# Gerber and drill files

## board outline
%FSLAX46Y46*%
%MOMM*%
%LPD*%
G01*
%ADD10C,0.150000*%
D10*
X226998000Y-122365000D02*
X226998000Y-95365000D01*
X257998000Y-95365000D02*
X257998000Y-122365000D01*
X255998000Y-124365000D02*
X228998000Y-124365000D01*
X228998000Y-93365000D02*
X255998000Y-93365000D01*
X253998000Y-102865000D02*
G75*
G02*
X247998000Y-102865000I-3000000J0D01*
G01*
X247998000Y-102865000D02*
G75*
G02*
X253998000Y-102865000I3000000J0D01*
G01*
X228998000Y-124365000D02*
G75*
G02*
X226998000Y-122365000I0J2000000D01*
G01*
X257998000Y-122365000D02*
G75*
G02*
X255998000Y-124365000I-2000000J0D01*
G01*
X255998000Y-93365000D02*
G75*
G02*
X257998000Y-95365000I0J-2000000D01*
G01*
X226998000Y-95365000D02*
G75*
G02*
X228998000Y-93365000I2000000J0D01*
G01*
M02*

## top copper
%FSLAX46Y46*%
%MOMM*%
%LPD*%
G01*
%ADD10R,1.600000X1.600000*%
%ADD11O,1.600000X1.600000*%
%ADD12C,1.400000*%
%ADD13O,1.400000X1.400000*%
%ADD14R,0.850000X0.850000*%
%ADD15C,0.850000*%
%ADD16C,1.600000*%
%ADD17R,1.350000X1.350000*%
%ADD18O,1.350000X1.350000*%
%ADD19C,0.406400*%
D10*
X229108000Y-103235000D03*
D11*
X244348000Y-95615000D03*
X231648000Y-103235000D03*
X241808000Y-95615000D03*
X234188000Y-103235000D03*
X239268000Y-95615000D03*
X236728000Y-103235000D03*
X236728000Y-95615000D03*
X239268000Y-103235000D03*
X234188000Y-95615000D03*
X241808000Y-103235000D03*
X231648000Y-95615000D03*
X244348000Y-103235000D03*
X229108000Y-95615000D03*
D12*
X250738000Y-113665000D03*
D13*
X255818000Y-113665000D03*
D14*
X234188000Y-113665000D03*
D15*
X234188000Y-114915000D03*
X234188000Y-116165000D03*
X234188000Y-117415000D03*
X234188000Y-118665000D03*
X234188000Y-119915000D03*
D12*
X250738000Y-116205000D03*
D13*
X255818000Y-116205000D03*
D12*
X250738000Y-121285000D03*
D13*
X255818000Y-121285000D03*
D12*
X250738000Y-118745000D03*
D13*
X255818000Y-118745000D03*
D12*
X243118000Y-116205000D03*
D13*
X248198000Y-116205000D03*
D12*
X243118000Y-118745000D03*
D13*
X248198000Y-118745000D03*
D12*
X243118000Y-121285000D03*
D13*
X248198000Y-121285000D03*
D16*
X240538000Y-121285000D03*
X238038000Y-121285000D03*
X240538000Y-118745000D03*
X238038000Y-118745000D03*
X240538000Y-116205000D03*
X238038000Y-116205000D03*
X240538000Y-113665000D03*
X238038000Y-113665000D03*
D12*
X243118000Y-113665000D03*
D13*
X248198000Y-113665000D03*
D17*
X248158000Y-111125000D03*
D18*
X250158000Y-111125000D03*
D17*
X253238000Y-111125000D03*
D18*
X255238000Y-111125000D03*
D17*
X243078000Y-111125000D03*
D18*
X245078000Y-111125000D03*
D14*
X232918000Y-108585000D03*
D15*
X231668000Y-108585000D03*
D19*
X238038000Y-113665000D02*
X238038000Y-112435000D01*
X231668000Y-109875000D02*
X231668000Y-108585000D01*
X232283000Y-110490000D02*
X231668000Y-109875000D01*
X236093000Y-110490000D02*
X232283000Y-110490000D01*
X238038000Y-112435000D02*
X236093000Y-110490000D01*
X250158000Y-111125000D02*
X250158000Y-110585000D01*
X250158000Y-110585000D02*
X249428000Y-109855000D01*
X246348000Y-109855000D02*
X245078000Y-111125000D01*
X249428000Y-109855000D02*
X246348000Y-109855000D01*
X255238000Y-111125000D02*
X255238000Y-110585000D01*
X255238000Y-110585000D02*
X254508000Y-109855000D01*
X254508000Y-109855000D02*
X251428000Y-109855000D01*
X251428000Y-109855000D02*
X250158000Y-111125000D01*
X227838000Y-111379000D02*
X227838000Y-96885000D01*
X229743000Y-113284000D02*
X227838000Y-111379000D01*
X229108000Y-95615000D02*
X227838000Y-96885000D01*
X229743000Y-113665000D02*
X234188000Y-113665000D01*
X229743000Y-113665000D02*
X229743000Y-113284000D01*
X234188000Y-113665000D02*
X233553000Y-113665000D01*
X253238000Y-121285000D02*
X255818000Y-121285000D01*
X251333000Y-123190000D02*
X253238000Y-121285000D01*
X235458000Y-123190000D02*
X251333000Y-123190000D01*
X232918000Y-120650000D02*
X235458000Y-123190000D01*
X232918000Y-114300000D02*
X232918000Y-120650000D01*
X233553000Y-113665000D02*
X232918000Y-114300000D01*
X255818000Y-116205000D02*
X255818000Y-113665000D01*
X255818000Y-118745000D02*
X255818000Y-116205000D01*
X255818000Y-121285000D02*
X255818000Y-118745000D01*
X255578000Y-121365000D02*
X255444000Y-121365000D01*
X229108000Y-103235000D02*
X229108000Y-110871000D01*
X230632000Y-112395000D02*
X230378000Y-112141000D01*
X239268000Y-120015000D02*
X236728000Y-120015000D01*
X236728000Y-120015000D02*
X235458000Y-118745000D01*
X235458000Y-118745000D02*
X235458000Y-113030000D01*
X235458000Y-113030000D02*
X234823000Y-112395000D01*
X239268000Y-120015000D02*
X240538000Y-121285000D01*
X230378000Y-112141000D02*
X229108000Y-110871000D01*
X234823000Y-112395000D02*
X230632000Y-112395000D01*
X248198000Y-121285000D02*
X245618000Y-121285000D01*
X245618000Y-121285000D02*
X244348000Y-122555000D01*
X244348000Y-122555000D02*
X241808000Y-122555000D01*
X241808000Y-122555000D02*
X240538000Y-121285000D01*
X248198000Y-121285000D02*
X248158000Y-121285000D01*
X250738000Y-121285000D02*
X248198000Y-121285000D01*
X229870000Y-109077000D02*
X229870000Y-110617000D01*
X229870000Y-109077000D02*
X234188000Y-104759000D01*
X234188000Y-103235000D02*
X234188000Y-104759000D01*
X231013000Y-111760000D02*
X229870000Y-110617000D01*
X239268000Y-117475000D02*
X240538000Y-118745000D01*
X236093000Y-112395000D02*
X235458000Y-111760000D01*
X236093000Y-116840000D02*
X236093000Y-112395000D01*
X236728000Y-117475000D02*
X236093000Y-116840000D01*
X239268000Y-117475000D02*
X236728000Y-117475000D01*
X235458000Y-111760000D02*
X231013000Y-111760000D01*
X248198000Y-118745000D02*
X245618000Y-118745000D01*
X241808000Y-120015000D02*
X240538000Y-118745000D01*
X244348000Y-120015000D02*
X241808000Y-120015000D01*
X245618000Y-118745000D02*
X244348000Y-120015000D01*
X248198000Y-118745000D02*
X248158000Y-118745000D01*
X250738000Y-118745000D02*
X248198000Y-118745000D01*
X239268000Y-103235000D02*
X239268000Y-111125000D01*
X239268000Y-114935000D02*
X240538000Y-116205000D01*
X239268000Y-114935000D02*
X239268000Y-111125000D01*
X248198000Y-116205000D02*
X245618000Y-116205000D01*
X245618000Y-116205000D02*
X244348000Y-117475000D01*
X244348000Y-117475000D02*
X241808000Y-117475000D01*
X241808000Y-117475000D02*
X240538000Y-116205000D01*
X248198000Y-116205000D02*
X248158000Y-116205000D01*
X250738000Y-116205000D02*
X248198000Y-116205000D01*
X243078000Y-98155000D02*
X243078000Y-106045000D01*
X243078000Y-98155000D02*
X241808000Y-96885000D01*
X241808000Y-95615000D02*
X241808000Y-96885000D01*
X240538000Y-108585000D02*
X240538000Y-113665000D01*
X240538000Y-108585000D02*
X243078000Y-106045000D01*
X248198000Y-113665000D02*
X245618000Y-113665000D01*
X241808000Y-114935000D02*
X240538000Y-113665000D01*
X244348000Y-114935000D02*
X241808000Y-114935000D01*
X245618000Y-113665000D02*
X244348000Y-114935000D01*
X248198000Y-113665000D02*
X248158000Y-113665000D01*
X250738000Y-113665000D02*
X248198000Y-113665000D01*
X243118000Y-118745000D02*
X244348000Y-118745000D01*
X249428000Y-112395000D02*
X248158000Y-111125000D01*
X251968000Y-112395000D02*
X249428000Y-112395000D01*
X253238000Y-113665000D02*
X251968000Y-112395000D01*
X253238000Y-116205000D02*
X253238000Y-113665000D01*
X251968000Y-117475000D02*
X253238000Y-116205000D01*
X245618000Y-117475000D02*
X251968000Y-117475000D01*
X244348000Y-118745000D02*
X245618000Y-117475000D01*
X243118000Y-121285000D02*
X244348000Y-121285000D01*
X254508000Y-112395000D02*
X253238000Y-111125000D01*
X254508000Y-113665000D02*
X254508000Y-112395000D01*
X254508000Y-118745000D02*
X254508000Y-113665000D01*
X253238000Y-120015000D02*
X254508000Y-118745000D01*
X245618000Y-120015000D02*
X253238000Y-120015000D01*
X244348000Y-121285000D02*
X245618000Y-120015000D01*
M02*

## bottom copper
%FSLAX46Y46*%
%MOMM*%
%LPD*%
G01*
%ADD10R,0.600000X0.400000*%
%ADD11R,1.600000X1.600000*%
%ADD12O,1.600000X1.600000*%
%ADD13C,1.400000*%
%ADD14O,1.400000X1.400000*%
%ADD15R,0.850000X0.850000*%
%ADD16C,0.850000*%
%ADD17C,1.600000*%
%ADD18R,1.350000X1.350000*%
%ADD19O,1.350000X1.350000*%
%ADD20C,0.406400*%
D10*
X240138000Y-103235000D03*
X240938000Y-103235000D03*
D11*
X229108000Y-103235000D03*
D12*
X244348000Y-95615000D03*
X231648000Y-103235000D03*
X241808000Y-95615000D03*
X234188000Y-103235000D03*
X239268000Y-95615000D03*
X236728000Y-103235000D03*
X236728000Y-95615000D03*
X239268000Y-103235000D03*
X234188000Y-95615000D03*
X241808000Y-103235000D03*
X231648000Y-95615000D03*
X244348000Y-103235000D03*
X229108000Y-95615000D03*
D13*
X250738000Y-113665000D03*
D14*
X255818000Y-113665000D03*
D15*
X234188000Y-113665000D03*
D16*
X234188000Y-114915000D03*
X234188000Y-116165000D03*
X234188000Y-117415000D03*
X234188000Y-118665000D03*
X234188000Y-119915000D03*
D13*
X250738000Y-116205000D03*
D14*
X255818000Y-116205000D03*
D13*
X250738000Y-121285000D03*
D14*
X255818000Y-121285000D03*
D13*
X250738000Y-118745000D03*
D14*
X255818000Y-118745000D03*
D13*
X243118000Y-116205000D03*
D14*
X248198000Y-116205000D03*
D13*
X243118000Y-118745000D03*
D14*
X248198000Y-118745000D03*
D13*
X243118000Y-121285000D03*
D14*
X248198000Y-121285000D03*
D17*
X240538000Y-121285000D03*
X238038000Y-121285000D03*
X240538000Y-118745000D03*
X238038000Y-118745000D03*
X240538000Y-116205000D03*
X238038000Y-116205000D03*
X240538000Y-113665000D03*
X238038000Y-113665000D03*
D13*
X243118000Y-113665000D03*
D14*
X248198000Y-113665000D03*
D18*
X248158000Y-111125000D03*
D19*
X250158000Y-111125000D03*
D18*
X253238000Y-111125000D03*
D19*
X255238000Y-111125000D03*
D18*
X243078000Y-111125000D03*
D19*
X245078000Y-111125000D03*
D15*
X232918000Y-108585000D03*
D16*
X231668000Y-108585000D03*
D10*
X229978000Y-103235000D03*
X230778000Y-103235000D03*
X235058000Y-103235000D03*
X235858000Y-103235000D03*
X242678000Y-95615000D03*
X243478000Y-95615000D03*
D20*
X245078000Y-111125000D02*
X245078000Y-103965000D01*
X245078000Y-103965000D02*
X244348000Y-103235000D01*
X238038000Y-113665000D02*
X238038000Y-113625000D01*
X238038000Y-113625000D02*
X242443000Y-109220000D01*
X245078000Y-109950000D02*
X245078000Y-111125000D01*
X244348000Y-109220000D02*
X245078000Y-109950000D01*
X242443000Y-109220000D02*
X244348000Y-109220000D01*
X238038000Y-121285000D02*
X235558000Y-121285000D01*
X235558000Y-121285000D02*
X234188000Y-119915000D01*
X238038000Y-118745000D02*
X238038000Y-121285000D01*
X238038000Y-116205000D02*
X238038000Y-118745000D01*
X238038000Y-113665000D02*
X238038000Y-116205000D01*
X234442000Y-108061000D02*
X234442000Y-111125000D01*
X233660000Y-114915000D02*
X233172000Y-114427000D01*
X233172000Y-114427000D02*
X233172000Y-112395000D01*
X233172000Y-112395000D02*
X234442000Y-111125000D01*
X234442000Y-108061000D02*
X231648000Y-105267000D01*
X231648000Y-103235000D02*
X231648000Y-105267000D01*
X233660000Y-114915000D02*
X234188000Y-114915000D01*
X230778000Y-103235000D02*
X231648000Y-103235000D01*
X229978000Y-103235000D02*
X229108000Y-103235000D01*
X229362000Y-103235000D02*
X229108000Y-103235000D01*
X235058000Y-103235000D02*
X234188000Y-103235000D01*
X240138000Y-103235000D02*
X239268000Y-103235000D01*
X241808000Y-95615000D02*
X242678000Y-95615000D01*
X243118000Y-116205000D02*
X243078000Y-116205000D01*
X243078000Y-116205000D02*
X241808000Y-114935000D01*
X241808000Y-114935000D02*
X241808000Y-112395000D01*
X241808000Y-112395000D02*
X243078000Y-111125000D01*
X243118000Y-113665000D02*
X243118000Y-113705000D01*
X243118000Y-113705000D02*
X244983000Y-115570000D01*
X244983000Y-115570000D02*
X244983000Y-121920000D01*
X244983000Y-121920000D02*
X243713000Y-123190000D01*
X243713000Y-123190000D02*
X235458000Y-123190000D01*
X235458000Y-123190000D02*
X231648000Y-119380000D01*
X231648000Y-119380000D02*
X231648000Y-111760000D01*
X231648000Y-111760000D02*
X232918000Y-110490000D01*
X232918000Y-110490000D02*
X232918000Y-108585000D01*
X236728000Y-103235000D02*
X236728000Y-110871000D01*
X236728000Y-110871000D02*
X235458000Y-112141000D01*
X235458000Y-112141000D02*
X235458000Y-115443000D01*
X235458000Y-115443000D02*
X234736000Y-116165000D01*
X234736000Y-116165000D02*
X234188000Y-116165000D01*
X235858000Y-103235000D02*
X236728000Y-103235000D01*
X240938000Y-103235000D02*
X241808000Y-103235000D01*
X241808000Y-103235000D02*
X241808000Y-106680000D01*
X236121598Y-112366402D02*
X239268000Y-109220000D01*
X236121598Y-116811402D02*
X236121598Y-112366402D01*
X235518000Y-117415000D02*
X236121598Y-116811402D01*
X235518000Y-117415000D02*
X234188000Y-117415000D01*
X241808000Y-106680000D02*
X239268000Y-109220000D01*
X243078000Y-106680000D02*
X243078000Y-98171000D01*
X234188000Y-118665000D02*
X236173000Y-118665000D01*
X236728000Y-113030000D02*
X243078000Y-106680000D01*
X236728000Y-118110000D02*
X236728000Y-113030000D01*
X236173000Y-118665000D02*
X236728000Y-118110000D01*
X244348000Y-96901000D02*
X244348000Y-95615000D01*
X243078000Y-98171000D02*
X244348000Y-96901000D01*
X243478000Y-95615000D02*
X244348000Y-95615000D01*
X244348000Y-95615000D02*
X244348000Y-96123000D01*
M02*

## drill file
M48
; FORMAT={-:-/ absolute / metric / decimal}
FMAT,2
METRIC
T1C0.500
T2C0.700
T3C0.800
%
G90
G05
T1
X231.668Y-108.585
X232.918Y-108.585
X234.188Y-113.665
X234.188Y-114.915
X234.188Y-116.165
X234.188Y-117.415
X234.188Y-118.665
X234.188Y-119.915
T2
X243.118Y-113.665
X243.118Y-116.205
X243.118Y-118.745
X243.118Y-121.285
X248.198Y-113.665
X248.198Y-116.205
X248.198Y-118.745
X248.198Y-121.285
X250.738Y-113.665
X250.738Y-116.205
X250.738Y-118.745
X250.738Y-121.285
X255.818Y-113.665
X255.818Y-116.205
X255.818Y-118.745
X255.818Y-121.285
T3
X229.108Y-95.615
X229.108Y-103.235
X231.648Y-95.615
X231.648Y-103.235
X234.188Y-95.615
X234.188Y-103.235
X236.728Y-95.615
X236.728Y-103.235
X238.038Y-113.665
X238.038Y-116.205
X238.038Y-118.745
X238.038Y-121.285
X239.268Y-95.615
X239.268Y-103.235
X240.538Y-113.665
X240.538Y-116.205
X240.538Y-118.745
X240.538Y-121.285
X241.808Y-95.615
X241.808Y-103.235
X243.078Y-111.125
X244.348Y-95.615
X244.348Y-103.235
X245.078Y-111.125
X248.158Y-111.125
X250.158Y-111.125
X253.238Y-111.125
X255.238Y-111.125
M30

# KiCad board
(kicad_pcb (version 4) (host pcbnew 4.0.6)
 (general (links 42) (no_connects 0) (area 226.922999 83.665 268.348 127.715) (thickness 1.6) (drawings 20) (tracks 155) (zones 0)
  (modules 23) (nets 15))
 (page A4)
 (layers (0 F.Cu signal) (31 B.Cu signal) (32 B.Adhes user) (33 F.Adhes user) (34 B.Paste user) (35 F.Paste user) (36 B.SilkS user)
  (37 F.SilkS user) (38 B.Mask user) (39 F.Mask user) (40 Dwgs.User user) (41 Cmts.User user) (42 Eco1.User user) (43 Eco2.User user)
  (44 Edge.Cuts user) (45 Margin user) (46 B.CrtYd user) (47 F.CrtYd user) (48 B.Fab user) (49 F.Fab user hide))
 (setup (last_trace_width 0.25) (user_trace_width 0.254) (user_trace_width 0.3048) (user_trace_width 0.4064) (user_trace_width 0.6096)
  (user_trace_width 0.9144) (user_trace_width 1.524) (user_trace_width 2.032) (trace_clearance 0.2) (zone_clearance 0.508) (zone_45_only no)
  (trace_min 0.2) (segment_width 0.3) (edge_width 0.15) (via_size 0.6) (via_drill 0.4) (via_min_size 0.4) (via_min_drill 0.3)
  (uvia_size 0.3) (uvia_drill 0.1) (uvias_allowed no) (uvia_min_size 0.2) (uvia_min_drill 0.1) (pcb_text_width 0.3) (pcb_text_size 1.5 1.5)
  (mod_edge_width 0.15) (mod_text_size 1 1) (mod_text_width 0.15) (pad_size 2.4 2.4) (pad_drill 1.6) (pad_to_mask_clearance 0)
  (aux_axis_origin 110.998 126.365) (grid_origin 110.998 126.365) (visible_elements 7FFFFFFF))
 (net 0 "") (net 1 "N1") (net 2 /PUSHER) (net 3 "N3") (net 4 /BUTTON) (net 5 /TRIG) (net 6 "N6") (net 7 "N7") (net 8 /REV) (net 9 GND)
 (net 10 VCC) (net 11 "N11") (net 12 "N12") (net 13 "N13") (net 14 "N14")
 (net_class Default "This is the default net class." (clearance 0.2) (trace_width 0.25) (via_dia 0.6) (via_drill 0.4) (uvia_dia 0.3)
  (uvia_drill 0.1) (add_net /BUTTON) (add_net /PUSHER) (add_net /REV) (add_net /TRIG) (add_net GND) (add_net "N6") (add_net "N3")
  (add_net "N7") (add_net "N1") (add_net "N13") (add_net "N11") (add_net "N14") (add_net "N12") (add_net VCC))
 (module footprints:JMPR (layer B.Cu) (at 240.538 103.235)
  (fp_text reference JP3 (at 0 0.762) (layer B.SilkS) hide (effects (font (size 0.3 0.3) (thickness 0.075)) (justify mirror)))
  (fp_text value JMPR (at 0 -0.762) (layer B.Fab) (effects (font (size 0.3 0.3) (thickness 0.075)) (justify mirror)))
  (pad 1 smd rect (at -0.4 0) (size 0.6 0.4) (layers B.Cu B.Paste B.Mask) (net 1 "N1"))
  (pad 2 smd rect (at 0.4 0) (size 0.6 0.4) (layers B.Cu B.Paste B.Mask) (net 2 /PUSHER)))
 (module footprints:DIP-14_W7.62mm (layer F.Cu) (at 229.108 103.235 90)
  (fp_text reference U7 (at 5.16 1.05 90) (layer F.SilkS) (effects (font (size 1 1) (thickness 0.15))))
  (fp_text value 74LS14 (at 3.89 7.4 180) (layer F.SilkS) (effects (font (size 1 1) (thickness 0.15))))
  (pad 1 thru_hole rect (at 0 0 90) (size 1.6 1.6) (drill 0.8) (layers *.Cu *.Mask) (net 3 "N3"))
  (pad 8 thru_hole oval (at 7.62 15.24 90) (size 1.6 1.6) (drill 0.8) (layers *.Cu *.Mask) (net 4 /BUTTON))
  (pad 2 thru_hole oval (at 0 2.54 90) (size 1.6 1.6) (drill 0.8) (layers *.Cu *.Mask) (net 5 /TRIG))
  (pad 9 thru_hole oval (at 7.62 12.7 90) (size 1.6 1.6) (drill 0.8) (layers *.Cu *.Mask) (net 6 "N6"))
  (pad 3 thru_hole oval (at 0 5.08 90) (size 1.6 1.6) (drill 0.8) (layers *.Cu *.Mask) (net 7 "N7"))
  (pad 10 thru_hole oval (at 7.62 10.16 90) (size 1.6 1.6) (drill 0.8) (layers *.Cu *.Mask))
  (pad 4 thru_hole oval (at 0 7.62 90) (size 1.6 1.6) (drill 0.8) (layers *.Cu *.Mask) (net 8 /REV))
  (pad 11 thru_hole oval (at 7.62 7.62 90) (size 1.6 1.6) (drill 0.8) (layers *.Cu *.Mask))
  (pad 5 thru_hole oval (at 0 10.16 90) (size 1.6 1.6) (drill 0.8) (layers *.Cu *.Mask) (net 1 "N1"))
  (pad 12 thru_hole oval (at 7.62 5.08 90) (size 1.6 1.6) (drill 0.8) (layers *.Cu *.Mask))
  (pad 6 thru_hole oval (at 0 12.7 90) (size 1.6 1.6) (drill 0.8) (layers *.Cu *.Mask) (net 2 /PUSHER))
  (pad 13 thru_hole oval (at 7.62 2.54 90) (size 1.6 1.6) (drill 0.8) (layers *.Cu *.Mask))
  (pad 7 thru_hole oval (at 0 15.24 90) (size 1.6 1.6) (drill 0.8) (layers *.Cu *.Mask) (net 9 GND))
  (pad 14 thru_hole oval (at 7.62 0 90) (size 1.6 1.6) (drill 0.8) (layers *.Cu *.Mask) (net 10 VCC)))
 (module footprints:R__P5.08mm (layer F.Cu) (at 253.238 113.665)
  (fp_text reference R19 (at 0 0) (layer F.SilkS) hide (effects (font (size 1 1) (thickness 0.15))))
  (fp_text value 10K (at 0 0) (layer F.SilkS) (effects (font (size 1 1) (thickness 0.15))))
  (pad 1 thru_hole circle (at -2.5 0) (size 1.4 1.4) (drill 0.7) (layers *.Cu *.Mask) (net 6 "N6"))
  (pad 2 thru_hole oval (at 2.58 0) (size 1.4 1.4) (drill 0.7) (layers *.Cu *.Mask) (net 10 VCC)))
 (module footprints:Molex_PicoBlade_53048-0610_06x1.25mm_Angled (layer F.Cu) (at 234.188 113.665 270)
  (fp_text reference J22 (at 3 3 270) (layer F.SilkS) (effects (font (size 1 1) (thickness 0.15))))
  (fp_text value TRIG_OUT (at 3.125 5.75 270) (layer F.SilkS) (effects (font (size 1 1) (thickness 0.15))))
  (pad 1 thru_hole rect (at 0 0 270) (size 0.85 0.85) (drill 0.5) (layers *.Cu *.Mask) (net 10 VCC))
  (pad 2 thru_hole circle (at 1.25 0 270) (size 0.85 0.85) (drill 0.5) (layers *.Cu *.Mask) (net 5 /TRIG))
  (pad 3 thru_hole circle (at 2.5 0 270) (size 0.85 0.85) (drill 0.5) (layers *.Cu *.Mask) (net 8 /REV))
  (pad 4 thru_hole circle (at 3.75 0 270) (size 0.85 0.85) (drill 0.5) (layers *.Cu *.Mask) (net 2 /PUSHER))
  (pad 5 thru_hole circle (at 5 0 270) (size 0.85 0.85) (drill 0.5) (layers *.Cu *.Mask) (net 4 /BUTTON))
  (pad 6 thru_hole circle (at 6.25 0 270) (size 0.85 0.85) (drill 0.5) (layers *.Cu *.Mask) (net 9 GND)))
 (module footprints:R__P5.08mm (layer F.Cu) (at 253.238 116.205)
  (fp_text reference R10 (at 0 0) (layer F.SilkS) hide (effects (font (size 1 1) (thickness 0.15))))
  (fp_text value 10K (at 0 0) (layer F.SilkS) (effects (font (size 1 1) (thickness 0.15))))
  (pad 1 thru_hole circle (at -2.5 0) (size 1.4 1.4) (drill 0.7) (layers *.Cu *.Mask) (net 1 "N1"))
  (pad 2 thru_hole oval (at 2.58 0) (size 1.4 1.4) (drill 0.7) (layers *.Cu *.Mask) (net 10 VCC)))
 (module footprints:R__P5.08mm (layer F.Cu) (at 253.238 121.285)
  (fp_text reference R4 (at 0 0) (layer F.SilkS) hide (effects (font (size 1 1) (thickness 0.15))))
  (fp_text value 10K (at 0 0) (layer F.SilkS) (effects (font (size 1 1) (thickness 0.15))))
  (pad 1 thru_hole circle (at -2.5 0) (size 1.4 1.4) (drill 0.7) (layers *.Cu *.Mask) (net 3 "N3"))
  (pad 2 thru_hole oval (at 2.58 0) (size 1.4 1.4) (drill 0.7) (layers *.Cu *.Mask) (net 10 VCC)))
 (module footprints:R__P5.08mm (layer F.Cu) (at 253.238 118.745)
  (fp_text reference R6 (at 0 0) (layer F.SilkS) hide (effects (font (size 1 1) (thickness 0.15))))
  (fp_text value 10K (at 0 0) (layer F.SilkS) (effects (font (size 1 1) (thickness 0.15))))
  (pad 1 thru_hole circle (at -2.5 0) (size 1.4 1.4) (drill 0.7) (layers *.Cu *.Mask) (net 7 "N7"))
  (pad 2 thru_hole oval (at 2.58 0) (size 1.4 1.4) (drill 0.7) (layers *.Cu *.Mask) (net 10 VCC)))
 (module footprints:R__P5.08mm (layer F.Cu) (at 245.618 116.205)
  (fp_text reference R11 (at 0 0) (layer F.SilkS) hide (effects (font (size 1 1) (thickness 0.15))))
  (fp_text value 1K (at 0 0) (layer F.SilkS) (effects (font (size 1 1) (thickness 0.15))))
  (pad 1 thru_hole circle (at -2.5 0) (size 1.4 1.4) (drill 0.7) (layers *.Cu *.Mask) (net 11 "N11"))
  (pad 2 thru_hole oval (at 2.58 0) (size 1.4 1.4) (drill 0.7) (layers *.Cu *.Mask) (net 1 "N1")))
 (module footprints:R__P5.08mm (layer F.Cu) (at 245.618 118.745)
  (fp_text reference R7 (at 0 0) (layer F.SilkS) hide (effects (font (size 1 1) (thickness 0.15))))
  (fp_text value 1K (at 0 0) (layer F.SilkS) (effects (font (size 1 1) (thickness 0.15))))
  (pad 1 thru_hole circle (at -2.5 0) (size 1.4 1.4) (drill 0.7) (layers *.Cu *.Mask) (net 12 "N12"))
  (pad 2 thru_hole oval (at 2.58 0) (size 1.4 1.4) (drill 0.7) (layers *.Cu *.Mask) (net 7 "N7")))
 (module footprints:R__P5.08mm (layer F.Cu) (at 245.618 121.285)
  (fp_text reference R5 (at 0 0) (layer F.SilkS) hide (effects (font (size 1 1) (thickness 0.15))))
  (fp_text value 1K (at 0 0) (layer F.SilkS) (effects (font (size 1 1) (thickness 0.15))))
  (pad 1 thru_hole circle (at -2.5 0) (size 1.4 1.4) (drill 0.7) (layers *.Cu *.Mask) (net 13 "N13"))
  (pad 2 thru_hole oval (at 2.58 0) (size 1.4 1.4) (drill 0.7) (layers *.Cu *.Mask) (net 3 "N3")))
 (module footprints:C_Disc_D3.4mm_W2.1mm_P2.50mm (layer F.Cu) (at 240.538 121.285 180)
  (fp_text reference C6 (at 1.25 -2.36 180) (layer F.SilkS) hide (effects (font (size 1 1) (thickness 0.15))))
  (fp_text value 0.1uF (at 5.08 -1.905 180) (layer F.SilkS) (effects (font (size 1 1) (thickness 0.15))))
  (pad 1 thru_hole circle (at 0 0 180) (size 1.6 1.6) (drill 0.8) (layers *.Cu *.Mask) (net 3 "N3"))
  (pad 2 thru_hole circle (at 2.5 0 180) (size 1.6 1.6) (drill 0.8) (layers *.Cu *.Mask) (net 9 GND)))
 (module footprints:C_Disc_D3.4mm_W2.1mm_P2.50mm (layer F.Cu) (at 240.538 118.745 180)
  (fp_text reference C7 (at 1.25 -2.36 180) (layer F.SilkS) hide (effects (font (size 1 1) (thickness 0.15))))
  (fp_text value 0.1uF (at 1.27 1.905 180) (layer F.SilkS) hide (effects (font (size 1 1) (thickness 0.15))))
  (pad 1 thru_hole circle (at 0 0 180) (size 1.6 1.6) (drill 0.8) (layers *.Cu *.Mask) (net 7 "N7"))
  (pad 2 thru_hole circle (at 2.5 0 180) (size 1.6 1.6) (drill 0.8) (layers *.Cu *.Mask) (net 9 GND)))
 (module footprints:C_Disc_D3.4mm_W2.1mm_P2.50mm (layer F.Cu) (at 240.538 116.205 180)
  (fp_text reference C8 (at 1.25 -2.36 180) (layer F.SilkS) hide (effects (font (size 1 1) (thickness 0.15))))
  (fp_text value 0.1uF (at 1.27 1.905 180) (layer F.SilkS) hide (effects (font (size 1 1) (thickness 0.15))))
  (pad 1 thru_hole circle (at 0 0 180) (size 1.6 1.6) (drill 0.8) (layers *.Cu *.Mask) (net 1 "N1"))
  (pad 2 thru_hole circle (at 2.5 0 180) (size 1.6 1.6) (drill 0.8) (layers *.Cu *.Mask) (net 9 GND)))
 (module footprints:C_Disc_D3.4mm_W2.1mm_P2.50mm (layer F.Cu) (at 240.538 113.665 180)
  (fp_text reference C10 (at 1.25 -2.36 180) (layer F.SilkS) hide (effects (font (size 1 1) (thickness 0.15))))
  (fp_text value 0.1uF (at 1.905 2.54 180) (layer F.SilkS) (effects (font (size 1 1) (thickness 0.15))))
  (pad 1 thru_hole circle (at 0 0 180) (size 1.6 1.6) (drill 0.8) (layers *.Cu *.Mask) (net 6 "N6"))
  (pad 2 thru_hole circle (at 2.5 0 180) (size 1.6 1.6) (drill 0.8) (layers *.Cu *.Mask) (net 9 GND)))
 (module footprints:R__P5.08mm (layer F.Cu) (at 245.618 113.665)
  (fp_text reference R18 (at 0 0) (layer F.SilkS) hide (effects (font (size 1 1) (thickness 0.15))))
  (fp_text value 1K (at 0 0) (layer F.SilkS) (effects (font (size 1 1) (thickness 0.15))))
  (pad 1 thru_hole circle (at -2.5 0) (size 1.4 1.4) (drill 0.7) (layers *.Cu *.Mask) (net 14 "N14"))
  (pad 2 thru_hole oval (at 2.58 0) (size 1.4 1.4) (drill 0.7) (layers *.Cu *.Mask) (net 6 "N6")))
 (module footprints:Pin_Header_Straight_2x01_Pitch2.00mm (layer F.Cu) (at 248.158 111.125)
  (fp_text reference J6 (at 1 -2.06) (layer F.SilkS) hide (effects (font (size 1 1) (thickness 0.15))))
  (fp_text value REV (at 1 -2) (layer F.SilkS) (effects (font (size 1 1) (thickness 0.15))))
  (pad 1 thru_hole rect (at 0 0) (size 1.35 1.35) (drill 0.8) (layers *.Cu *.Mask) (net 12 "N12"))
  (pad 2 thru_hole oval (at 2 0) (size 1.35 1.35) (drill 0.8) (layers *.Cu *.Mask) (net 9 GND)))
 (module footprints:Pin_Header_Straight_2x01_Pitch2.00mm (layer F.Cu) (at 253.238 111.125)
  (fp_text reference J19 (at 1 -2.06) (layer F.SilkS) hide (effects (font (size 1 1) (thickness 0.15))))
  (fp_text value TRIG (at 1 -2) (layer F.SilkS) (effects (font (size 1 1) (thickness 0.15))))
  (pad 1 thru_hole rect (at 0 0) (size 1.35 1.35) (drill 0.8) (layers *.Cu *.Mask) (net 13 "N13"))
  (pad 2 thru_hole oval (at 2 0) (size 1.35 1.35) (drill 0.8) (layers *.Cu *.Mask) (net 9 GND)))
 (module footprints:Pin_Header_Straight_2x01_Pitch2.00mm (layer F.Cu) (at 243.078 111.125)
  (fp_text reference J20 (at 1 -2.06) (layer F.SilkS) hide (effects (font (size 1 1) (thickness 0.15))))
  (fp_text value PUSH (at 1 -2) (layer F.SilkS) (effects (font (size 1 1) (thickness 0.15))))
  (pad 1 thru_hole rect (at 0 0) (size 1.35 1.35) (drill 0.8) (layers *.Cu *.Mask) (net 11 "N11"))
  (pad 2 thru_hole oval (at 2 0) (size 1.35 1.35) (drill 0.8) (layers *.Cu *.Mask) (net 9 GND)))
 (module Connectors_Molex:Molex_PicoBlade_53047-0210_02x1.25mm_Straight (layer F.Cu) (at 232.918 108.585 180)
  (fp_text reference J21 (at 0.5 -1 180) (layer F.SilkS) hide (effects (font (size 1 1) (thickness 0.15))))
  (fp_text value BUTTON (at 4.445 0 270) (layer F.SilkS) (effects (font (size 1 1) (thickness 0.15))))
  (pad 1 thru_hole rect (at 0 0 180) (size 0.85 0.85) (drill 0.5) (layers *.Cu *.Mask) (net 14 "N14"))
  (pad 2 thru_hole circle (at 1.25 0 180) (size 0.85 0.85) (drill 0.5) (layers *.Cu *.Mask) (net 9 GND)))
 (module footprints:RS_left (layer F.Cu) (at 240.03 106.537)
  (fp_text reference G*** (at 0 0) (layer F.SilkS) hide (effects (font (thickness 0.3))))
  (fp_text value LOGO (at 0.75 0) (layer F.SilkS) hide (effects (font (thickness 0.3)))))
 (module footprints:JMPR (layer B.Cu) (at 230.378 103.235)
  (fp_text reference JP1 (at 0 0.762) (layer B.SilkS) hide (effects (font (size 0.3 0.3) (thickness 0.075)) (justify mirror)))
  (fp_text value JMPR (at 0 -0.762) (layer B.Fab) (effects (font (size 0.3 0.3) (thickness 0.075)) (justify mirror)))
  (pad 1 smd rect (at -0.4 0) (size 0.6 0.4) (layers B.Cu B.Paste B.Mask) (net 3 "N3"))
  (pad 2 smd rect (at 0.4 0) (size 0.6 0.4) (layers B.Cu B.Paste B.Mask) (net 5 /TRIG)))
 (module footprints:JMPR (layer B.Cu) (at 235.458 103.235)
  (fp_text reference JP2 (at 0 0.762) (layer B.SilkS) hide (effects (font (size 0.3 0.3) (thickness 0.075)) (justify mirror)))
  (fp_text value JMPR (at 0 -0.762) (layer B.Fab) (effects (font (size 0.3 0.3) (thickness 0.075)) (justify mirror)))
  (pad 1 smd rect (at -0.4 0) (size 0.6 0.4) (layers B.Cu B.Paste B.Mask) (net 7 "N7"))
  (pad 2 smd rect (at 0.4 0) (size 0.6 0.4) (layers B.Cu B.Paste B.Mask) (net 8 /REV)))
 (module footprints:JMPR (layer B.Cu) (at 243.078 95.615)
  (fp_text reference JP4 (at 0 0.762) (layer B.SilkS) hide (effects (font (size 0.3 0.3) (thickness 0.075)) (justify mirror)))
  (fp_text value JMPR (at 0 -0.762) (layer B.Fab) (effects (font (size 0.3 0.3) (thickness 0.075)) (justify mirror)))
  (pad 1 smd rect (at -0.4 0) (size 0.6 0.4) (layers B.Cu B.Paste B.Mask) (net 6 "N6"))
  (pad 2 smd rect (at 0.4 0) (size 0.6 0.4) (layers B.Cu B.Paste B.Mask) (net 4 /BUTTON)))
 (gr_line (start 226.998 122.365) (end 226.998 95.365) (angle 90) (layer Edge.Cuts) (width 0.15))
 (gr_line (start 257.998 95.365) (end 257.998 122.365) (angle 90) (layer Edge.Cuts) (width 0.15))
 (gr_line (start 255.998 124.365) (end 228.998 124.365) (angle 90) (layer Edge.Cuts) (width 0.15))
 (gr_line (start 228.998 93.365) (end 255.998 93.365) (angle 90) (layer Edge.Cuts) (width 0.15))
 (gr_circle (center 250.998 102.865) (end 253.998 102.865) (layer Edge.Cuts) (width 0.15))
 (gr_arc (start 228.998 122.365) (end 228.998 124.365) (angle 90) (layer Edge.Cuts) (width 0.15))
 (gr_arc (start 255.998 122.365) (end 257.998 122.365) (angle 90) (layer Edge.Cuts) (width 0.15))
 (gr_arc (start 255.998 95.365) (end 255.998 93.365) (angle 90) (layer Edge.Cuts) (width 0.15))
 (gr_arc (start 228.998 95.365) (end 226.998 95.365) (angle 90) (layer Edge.Cuts) (width 0.15))
 (segment (start 245.078 111.125) (end 245.078 103.965) (width 0.4064) (layer B.Cu) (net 9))
 (segment (start 245.078 103.965) (end 244.348 103.235) (width 0.4064) (layer B.Cu) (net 9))
 (segment (start 238.038 113.665) (end 238.038 113.625) (width 0.4064) (layer B.Cu) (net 9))
 (segment (start 238.038 113.625) (end 242.443 109.22) (width 0.4064) (layer B.Cu) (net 9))
 (segment (start 245.078 109.95) (end 245.078 111.125) (width 0.4064) (layer B.Cu) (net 9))
 (segment (start 244.348 109.22) (end 245.078 109.95) (width 0.4064) (layer B.Cu) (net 9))
 (segment (start 242.443 109.22) (end 244.348 109.22) (width 0.4064) (layer B.Cu) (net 9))
 (segment (start 238.038 113.665) (end 238.038 112.435) (width 0.4064) (layer F.Cu) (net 9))
 (segment (start 231.668 109.875) (end 231.668 108.585) (width 0.4064) (layer F.Cu) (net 9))
 (segment (start 232.283 110.49) (end 231.668 109.875) (width 0.4064) (layer F.Cu) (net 9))
 (segment (start 236.093 110.49) (end 232.283 110.49) (width 0.4064) (layer F.Cu) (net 9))
 (segment (start 238.038 112.435) (end 236.093 110.49) (width 0.4064) (layer F.Cu) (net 9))
 (segment (start 250.158 111.125) (end 250.158 110.585) (width 0.4064) (layer F.Cu) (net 9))
 (segment (start 250.158 110.585) (end 249.428 109.855) (width 0.4064) (layer F.Cu) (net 9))
 (segment (start 246.348 109.855) (end 245.078 111.125) (width 0.4064) (layer F.Cu) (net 9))
 (segment (start 249.428 109.855) (end 246.348 109.855) (width 0.4064) (layer F.Cu) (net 9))
 (segment (start 255.238 111.125) (end 255.238 110.585) (width 0.4064) (layer F.Cu) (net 9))
 (segment (start 255.238 110.585) (end 254.508 109.855) (width 0.4064) (layer F.Cu) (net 9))
 (segment (start 254.508 109.855) (end 251.428 109.855) (width 0.4064) (layer F.Cu) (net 9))
 (segment (start 251.428 109.855) (end 250.158 111.125) (width 0.4064) (layer F.Cu) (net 9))
 (segment (start 238.038 121.285) (end 235.558 121.285) (width 0.4064) (layer B.Cu) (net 9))
 (segment (start 235.558 121.285) (end 234.188 119.915) (width 0.4064) (layer B.Cu) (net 9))
 (segment (start 238.038 118.745) (end 238.038 121.285) (width 0.4064) (layer B.Cu) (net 9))
 (segment (start 238.038 116.205) (end 238.038 118.745) (width 0.4064) (layer B.Cu) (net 9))
 (segment (start 238.038 113.665) (end 238.038 116.205) (width 0.4064) (layer B.Cu) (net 9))
 (segment (start 227.838 111.379) (end 227.838 96.885) (width 0.4064) (layer F.Cu) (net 10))
 (segment (start 229.743 113.284) (end 227.838 111.379) (width 0.4064) (layer F.Cu) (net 10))
 (segment (start 229.108 95.615) (end 227.838 96.885) (width 0.4064) (layer F.Cu) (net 10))
 (segment (start 229.743 113.665) (end 234.188 113.665) (width 0.4064) (layer F.Cu) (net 10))
 (segment (start 229.743 113.665) (end 229.743 113.284) (width 0.4064) (layer F.Cu) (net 10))
 (segment (start 234.188 113.665) (end 233.553 113.665) (width 0.4064) (layer F.Cu) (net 10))
 (segment (start 253.238 121.285) (end 255.818 121.285) (width 0.4064) (layer F.Cu) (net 10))
 (segment (start 251.333 123.19) (end 253.238 121.285) (width 0.4064) (layer F.Cu) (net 10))
 (segment (start 235.458 123.19) (end 251.333 123.19) (width 0.4064) (layer F.Cu) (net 10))
 (segment (start 232.918 120.65) (end 235.458 123.19) (width 0.4064) (layer F.Cu) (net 10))
 (segment (start 232.918 114.3) (end 232.918 120.65) (width 0.4064) (layer F.Cu) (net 10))
 (segment (start 233.553 113.665) (end 232.918 114.3) (width 0.4064) (layer F.Cu) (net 10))
 (segment (start 255.818 116.205) (end 255.818 113.665) (width 0.4064) (layer F.Cu) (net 10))
 (segment (start 255.818 118.745) (end 255.818 116.205) (width 0.4064) (layer F.Cu) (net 10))
 (segment (start 255.818 121.285) (end 255.818 118.745) (width 0.4064) (layer F.Cu) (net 10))
 (segment (start 255.578 121.365) (end 255.444 121.365) (width 0.4064) (layer F.Cu) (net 10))
 (segment (start 234.442 108.061) (end 234.442 111.125) (width 0.4064) (layer B.Cu) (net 5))
 (segment (start 233.66 114.915) (end 233.172 114.427) (width 0.4064) (layer B.Cu) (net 5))
 (segment (start 233.172 114.427) (end 233.172 112.395) (width 0.4064) (layer B.Cu) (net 5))
 (segment (start 233.172 112.395) (end 234.442 111.125) (width 0.4064) (layer B.Cu) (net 5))
 (segment (start 234.442 108.061) (end 231.648 105.267) (width 0.4064) (layer B.Cu) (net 5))
 (segment (start 231.648 103.235) (end 231.648 105.267) (width 0.4064) (layer B.Cu) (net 5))
 (segment (start 233.66 114.915) (end 234.188 114.915) (width 0.4064) (layer B.Cu) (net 5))
 (segment (start 230.778 103.235) (end 231.648 103.235) (width 0.4064) (layer B.Cu) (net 5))
 (segment (start 229.108 103.235) (end 229.108 110.871) (width 0.4064) (layer F.Cu) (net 3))
 (segment (start 230.632 112.395) (end 230.378 112.141) (width 0.4064) (layer F.Cu) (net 3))
 (segment (start 239.268 120.015) (end 236.728 120.015) (width 0.4064) (layer F.Cu) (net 3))
 (segment (start 236.728 120.015) (end 235.458 118.745) (width 0.4064) (layer F.Cu) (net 3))
 (segment (start 235.458 118.745) (end 235.458 113.03) (width 0.4064) (layer F.Cu) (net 3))
 (segment (start 235.458 113.03) (end 234.823 112.395) (width 0.4064) (layer F.Cu) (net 3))
 (segment (start 239.268 120.015) (end 240.538 121.285) (width 0.4064) (layer F.Cu) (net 3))
 (segment (start 230.378 112.141) (end 229.108 110.871) (width 0.4064) (layer F.Cu) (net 3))
 (segment (start 234.823 112.395) (end 230.632 112.395) (width 0.4064) (layer F.Cu) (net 3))
 (segment (start 229.978 103.235) (end 229.108 103.235) (width 0.4064) (layer B.Cu) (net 3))
 (segment (start 229.362 103.235) (end 229.108 103.235) (width 0.4064) (layer B.Cu) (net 3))
 (segment (start 248.198 121.285) (end 245.618 121.285) (width 0.4064) (layer F.Cu) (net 3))
 (segment (start 245.618 121.285) (end 244.348 122.555) (width 0.4064) (layer F.Cu) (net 3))
 (segment (start 244.348 122.555) (end 241.808 122.555) (width 0.4064) (layer F.Cu) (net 3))
 (segment (start 241.808 122.555) (end 240.538 121.285) (width 0.4064) (layer F.Cu) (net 3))
 (segment (start 248.198 121.285) (end 248.158 121.285) (width 0.4064) (layer F.Cu) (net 3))
 (segment (start 250.738 121.285) (end 248.198 121.285) (width 0.4064) (layer F.Cu) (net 3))
 (segment (start 229.87 109.077) (end 229.87 110.617) (width 0.4064) (layer F.Cu) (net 7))
 (segment (start 229.87 109.077) (end 234.188 104.759) (width 0.4064) (layer F.Cu) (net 7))
 (segment (start 234.188 103.235) (end 234.188 104.759) (width 0.4064) (layer F.Cu) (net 7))
 (segment (start 231.013 111.76) (end 229.87 110.617) (width 0.4064) (layer F.Cu) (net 7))
 (segment (start 239.268 117.475) (end 240.538 118.745) (width 0.4064) (layer F.Cu) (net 7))
 (segment (start 236.093 112.395) (end 235.458 111.76) (width 0.4064) (layer F.Cu) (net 7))
 (segment (start 236.093 116.84) (end 236.093 112.395) (width 0.4064) (layer F.Cu) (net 7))
 (segment (start 236.728 117.475) (end 236.093 116.84) (width 0.4064) (layer F.Cu) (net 7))
 (segment (start 239.268 117.475) (end 236.728 117.475) (width 0.4064) (layer F.Cu) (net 7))
 (segment (start 235.458 111.76) (end 231.013 111.76) (width 0.4064) (layer F.Cu) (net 7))
 (segment (start 235.058 103.235) (end 234.188 103.235) (width 0.4064) (layer B.Cu) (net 7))
 (segment (start 248.198 118.745) (end 245.618 118.745) (width 0.4064) (layer F.Cu) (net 7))
 (segment (start 241.808 120.015) (end 240.538 118.745) (width 0.4064) (layer F.Cu) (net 7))
 (segment (start 244.348 120.015) (end 241.808 120.015) (width 0.4064) (layer F.Cu) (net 7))
 (segment (start 245.618 118.745) (end 244.348 120.015) (width 0.4064) (layer F.Cu) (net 7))
 (segment (start 248.198 118.745) (end 248.158 118.745) (width 0.4064) (layer F.Cu) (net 7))
 (segment (start 250.738 118.745) (end 248.198 118.745) (width 0.4064) (layer F.Cu) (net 7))
 (segment (start 239.268 103.235) (end 239.268 111.125) (width 0.4064) (layer F.Cu) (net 1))
 (segment (start 239.268 114.935) (end 240.538 116.205) (width 0.4064) (layer F.Cu) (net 1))
 (segment (start 239.268 114.935) (end 239.268 111.125) (width 0.4064) (layer F.Cu) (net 1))
 (segment (start 240.138 103.235) (end 239.268 103.235) (width 0.4064) (layer B.Cu) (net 1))
 (segment (start 248.198 116.205) (end 245.618 116.205) (width 0.4064) (layer F.Cu) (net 1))
 (segment (start 245.618 116.205) (end 244.348 117.475) (width 0.4064) (layer F.Cu) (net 1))
 (segment (start 244.348 117.475) (end 241.808 117.475) (width 0.4064) (layer F.Cu) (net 1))
 (segment (start 241.808 117.475) (end 240.538 116.205) (width 0.4064) (layer F.Cu) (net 1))
 (segment (start 248.198 116.205) (end 248.158 116.205) (width 0.4064) (layer F.Cu) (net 1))
 (segment (start 250.738 116.205) (end 248.198 116.205) (width 0.4064) (layer F.Cu) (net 1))
 (segment (start 243.078 98.155) (end 243.078 106.045) (width 0.4064) (layer F.Cu) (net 6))
 (segment (start 243.078 98.155) (end 241.808 96.885) (width 0.4064) (layer F.Cu) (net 6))
 (segment (start 241.808 95.615) (end 241.808 96.885) (width 0.4064) (layer F.Cu) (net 6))
 (segment (start 240.538 108.585) (end 240.538 113.665) (width 0.4064) (layer F.Cu) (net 6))
 (segment (start 240.538 108.585) (end 243.078 106.045) (width 0.4064) (layer F.Cu) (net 6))
 (segment (start 241.808 95.615) (end 242.678 95.615) (width 0.4064) (layer B.Cu) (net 6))
 (segment (start 248.198 113.665) (end 245.618 113.665) (width 0.4064) (layer F.Cu) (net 6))
 (segment (start 241.808 114.935) (end 240.538 113.665) (width 0.4064) (layer F.Cu) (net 6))
 (segment (start 244.348 114.935) (end 241.808 114.935) (width 0.4064) (layer F.Cu) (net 6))
 (segment (start 245.618 113.665) (end 244.348 114.935) (width 0.4064) (layer F.Cu) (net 6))
 (segment (start 248.198 113.665) (end 248.158 113.665) (width 0.4064) (layer F.Cu) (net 6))
 (segment (start 250.738 113.665) (end 248.198 113.665) (width 0.4064) (layer F.Cu) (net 6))
 (segment (start 243.118 118.745) (end 244.348 118.745) (width 0.4064) (layer F.Cu) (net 12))
 (segment (start 249.428 112.395) (end 248.158 111.125) (width 0.4064) (layer F.Cu) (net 12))
 (segment (start 251.968 112.395) (end 249.428 112.395) (width 0.4064) (layer F.Cu) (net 12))
 (segment (start 253.238 113.665) (end 251.968 112.395) (width 0.4064) (layer F.Cu) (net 12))
 (segment (start 253.238 116.205) (end 253.238 113.665) (width 0.4064) (layer F.Cu) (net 12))
 (segment (start 251.968 117.475) (end 253.238 116.205) (width 0.4064) (layer F.Cu) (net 12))
 (segment (start 245.618 117.475) (end 251.968 117.475) (width 0.4064) (layer F.Cu) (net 12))
 (segment (start 244.348 118.745) (end 245.618 117.475) (width 0.4064) (layer F.Cu) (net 12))
 (segment (start 243.118 121.285) (end 244.348 121.285) (width 0.4064) (layer F.Cu) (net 13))
 (segment (start 254.508 112.395) (end 253.238 111.125) (width 0.4064) (layer F.Cu) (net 13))
 (segment (start 254.508 113.665) (end 254.508 112.395) (width 0.4064) (layer F.Cu) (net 13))
 (segment (start 254.508 118.745) (end 254.508 113.665) (width 0.4064) (layer F.Cu) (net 13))
 (segment (start 253.238 120.015) (end 254.508 118.745) (width 0.4064) (layer F.Cu) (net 13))
 (segment (start 245.618 120.015) (end 253.238 120.015) (width 0.4064) (layer F.Cu) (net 13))
 (segment (start 244.348 121.285) (end 245.618 120.015) (width 0.4064) (layer F.Cu) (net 13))
 (segment (start 243.118 116.205) (end 243.078 116.205) (width 0.4064) (layer B.Cu) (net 11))
 (segment (start 243.078 116.205) (end 241.808 114.935) (width 0.4064) (layer B.Cu) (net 11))
 (segment (start 241.808 114.935) (end 241.808 112.395) (width 0.4064) (layer B.Cu) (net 11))
 (segment (start 241.808 112.395) (end 243.078 111.125) (width 0.4064) (layer B.Cu) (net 11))
 (segment (start 243.118 113.665) (end 243.118 113.705) (width 0.4064) (layer B.Cu) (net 14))
 (segment (start 243.118 113.705) (end 244.983 115.57) (width 0.4064) (layer B.Cu) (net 14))
 (segment (start 244.983 115.57) (end 244.983 121.92) (width 0.4064) (layer B.Cu) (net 14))
 (segment (start 244.983 121.92) (end 243.713 123.19) (width 0.4064) (layer B.Cu) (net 14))
 (segment (start 243.713 123.19) (end 235.458 123.19) (width 0.4064) (layer B.Cu) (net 14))
 (segment (start 235.458 123.19) (end 231.648 119.38) (width 0.4064) (layer B.Cu) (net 14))
 (segment (start 231.648 119.38) (end 231.648 111.76) (width 0.4064) (layer B.Cu) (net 14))
 (segment (start 231.648 111.76) (end 232.918 110.49) (width 0.4064) (layer B.Cu) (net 14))
 (segment (start 232.918 110.49) (end 232.918 108.585) (width 0.4064) (layer B.Cu) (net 14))
 (segment (start 236.728 103.235) (end 236.728 110.871) (width 0.4064) (layer B.Cu) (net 8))
 (segment (start 236.728 110.871) (end 235.458 112.141) (width 0.4064) (layer B.Cu) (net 8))
 (segment (start 235.458 112.141) (end 235.458 115.443) (width 0.4064) (layer B.Cu) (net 8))
 (segment (start 235.458 115.443) (end 234.736 116.165) (width 0.4064) (layer B.Cu) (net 8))
 (segment (start 234.736 116.165) (end 234.188 116.165) (width 0.4064) (layer B.Cu) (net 8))
 (segment (start 235.858 103.235) (end 236.728 103.235) (width 0.4064) (layer B.Cu) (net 8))
 (segment (start 240.938 103.235) (end 241.808 103.235) (width 0.4064) (layer B.Cu) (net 2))
 (segment (start 241.808 103.235) (end 241.808 106.68) (width 0.4064) (layer B.Cu) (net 2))
 (segment (start 236.121598 112.366402) (end 239.268 109.22) (width 0.4064) (layer B.Cu) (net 2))
 (segment (start 236.121598 116.811402) (end 236.121598 112.366402) (width 0.4064) (layer B.Cu) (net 2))
 (segment (start 235.518 117.415) (end 236.121598 116.811402) (width 0.4064) (layer B.Cu) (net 2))
 (segment (start 235.518 117.415) (end 234.188 117.415) (width 0.4064) (layer B.Cu) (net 2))
 (segment (start 241.808 106.68) (end 239.268 109.22) (width 0.4064) (layer B.Cu) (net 2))
 (segment (start 243.078 106.68) (end 243.078 98.171) (width 0.4064) (layer B.Cu) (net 4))
 (segment (start 234.188 118.665) (end 236.173 118.665) (width 0.4064) (layer B.Cu) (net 4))
 (segment (start 236.728 113.03) (end 243.078 106.68) (width 0.4064) (layer B.Cu) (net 4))
 (segment (start 236.728 118.11) (end 236.728 113.03) (width 0.4064) (layer B.Cu) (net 4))
 (segment (start 236.173 118.665) (end 236.728 118.11) (width 0.4064) (layer B.Cu) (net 4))
 (segment (start 244.348 96.901) (end 244.348 95.615) (width 0.4064) (layer B.Cu) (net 4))
 (segment (start 243.078 98.171) (end 244.348 96.901) (width 0.4064) (layer B.Cu) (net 4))
 (segment (start 243.478 95.615) (end 244.348 95.615) (width 0.4064) (layer B.Cu) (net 4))
 (segment (start 244.348 95.615) (end 244.348 96.123) (width 0.4064) (layer B.Cu) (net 4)))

